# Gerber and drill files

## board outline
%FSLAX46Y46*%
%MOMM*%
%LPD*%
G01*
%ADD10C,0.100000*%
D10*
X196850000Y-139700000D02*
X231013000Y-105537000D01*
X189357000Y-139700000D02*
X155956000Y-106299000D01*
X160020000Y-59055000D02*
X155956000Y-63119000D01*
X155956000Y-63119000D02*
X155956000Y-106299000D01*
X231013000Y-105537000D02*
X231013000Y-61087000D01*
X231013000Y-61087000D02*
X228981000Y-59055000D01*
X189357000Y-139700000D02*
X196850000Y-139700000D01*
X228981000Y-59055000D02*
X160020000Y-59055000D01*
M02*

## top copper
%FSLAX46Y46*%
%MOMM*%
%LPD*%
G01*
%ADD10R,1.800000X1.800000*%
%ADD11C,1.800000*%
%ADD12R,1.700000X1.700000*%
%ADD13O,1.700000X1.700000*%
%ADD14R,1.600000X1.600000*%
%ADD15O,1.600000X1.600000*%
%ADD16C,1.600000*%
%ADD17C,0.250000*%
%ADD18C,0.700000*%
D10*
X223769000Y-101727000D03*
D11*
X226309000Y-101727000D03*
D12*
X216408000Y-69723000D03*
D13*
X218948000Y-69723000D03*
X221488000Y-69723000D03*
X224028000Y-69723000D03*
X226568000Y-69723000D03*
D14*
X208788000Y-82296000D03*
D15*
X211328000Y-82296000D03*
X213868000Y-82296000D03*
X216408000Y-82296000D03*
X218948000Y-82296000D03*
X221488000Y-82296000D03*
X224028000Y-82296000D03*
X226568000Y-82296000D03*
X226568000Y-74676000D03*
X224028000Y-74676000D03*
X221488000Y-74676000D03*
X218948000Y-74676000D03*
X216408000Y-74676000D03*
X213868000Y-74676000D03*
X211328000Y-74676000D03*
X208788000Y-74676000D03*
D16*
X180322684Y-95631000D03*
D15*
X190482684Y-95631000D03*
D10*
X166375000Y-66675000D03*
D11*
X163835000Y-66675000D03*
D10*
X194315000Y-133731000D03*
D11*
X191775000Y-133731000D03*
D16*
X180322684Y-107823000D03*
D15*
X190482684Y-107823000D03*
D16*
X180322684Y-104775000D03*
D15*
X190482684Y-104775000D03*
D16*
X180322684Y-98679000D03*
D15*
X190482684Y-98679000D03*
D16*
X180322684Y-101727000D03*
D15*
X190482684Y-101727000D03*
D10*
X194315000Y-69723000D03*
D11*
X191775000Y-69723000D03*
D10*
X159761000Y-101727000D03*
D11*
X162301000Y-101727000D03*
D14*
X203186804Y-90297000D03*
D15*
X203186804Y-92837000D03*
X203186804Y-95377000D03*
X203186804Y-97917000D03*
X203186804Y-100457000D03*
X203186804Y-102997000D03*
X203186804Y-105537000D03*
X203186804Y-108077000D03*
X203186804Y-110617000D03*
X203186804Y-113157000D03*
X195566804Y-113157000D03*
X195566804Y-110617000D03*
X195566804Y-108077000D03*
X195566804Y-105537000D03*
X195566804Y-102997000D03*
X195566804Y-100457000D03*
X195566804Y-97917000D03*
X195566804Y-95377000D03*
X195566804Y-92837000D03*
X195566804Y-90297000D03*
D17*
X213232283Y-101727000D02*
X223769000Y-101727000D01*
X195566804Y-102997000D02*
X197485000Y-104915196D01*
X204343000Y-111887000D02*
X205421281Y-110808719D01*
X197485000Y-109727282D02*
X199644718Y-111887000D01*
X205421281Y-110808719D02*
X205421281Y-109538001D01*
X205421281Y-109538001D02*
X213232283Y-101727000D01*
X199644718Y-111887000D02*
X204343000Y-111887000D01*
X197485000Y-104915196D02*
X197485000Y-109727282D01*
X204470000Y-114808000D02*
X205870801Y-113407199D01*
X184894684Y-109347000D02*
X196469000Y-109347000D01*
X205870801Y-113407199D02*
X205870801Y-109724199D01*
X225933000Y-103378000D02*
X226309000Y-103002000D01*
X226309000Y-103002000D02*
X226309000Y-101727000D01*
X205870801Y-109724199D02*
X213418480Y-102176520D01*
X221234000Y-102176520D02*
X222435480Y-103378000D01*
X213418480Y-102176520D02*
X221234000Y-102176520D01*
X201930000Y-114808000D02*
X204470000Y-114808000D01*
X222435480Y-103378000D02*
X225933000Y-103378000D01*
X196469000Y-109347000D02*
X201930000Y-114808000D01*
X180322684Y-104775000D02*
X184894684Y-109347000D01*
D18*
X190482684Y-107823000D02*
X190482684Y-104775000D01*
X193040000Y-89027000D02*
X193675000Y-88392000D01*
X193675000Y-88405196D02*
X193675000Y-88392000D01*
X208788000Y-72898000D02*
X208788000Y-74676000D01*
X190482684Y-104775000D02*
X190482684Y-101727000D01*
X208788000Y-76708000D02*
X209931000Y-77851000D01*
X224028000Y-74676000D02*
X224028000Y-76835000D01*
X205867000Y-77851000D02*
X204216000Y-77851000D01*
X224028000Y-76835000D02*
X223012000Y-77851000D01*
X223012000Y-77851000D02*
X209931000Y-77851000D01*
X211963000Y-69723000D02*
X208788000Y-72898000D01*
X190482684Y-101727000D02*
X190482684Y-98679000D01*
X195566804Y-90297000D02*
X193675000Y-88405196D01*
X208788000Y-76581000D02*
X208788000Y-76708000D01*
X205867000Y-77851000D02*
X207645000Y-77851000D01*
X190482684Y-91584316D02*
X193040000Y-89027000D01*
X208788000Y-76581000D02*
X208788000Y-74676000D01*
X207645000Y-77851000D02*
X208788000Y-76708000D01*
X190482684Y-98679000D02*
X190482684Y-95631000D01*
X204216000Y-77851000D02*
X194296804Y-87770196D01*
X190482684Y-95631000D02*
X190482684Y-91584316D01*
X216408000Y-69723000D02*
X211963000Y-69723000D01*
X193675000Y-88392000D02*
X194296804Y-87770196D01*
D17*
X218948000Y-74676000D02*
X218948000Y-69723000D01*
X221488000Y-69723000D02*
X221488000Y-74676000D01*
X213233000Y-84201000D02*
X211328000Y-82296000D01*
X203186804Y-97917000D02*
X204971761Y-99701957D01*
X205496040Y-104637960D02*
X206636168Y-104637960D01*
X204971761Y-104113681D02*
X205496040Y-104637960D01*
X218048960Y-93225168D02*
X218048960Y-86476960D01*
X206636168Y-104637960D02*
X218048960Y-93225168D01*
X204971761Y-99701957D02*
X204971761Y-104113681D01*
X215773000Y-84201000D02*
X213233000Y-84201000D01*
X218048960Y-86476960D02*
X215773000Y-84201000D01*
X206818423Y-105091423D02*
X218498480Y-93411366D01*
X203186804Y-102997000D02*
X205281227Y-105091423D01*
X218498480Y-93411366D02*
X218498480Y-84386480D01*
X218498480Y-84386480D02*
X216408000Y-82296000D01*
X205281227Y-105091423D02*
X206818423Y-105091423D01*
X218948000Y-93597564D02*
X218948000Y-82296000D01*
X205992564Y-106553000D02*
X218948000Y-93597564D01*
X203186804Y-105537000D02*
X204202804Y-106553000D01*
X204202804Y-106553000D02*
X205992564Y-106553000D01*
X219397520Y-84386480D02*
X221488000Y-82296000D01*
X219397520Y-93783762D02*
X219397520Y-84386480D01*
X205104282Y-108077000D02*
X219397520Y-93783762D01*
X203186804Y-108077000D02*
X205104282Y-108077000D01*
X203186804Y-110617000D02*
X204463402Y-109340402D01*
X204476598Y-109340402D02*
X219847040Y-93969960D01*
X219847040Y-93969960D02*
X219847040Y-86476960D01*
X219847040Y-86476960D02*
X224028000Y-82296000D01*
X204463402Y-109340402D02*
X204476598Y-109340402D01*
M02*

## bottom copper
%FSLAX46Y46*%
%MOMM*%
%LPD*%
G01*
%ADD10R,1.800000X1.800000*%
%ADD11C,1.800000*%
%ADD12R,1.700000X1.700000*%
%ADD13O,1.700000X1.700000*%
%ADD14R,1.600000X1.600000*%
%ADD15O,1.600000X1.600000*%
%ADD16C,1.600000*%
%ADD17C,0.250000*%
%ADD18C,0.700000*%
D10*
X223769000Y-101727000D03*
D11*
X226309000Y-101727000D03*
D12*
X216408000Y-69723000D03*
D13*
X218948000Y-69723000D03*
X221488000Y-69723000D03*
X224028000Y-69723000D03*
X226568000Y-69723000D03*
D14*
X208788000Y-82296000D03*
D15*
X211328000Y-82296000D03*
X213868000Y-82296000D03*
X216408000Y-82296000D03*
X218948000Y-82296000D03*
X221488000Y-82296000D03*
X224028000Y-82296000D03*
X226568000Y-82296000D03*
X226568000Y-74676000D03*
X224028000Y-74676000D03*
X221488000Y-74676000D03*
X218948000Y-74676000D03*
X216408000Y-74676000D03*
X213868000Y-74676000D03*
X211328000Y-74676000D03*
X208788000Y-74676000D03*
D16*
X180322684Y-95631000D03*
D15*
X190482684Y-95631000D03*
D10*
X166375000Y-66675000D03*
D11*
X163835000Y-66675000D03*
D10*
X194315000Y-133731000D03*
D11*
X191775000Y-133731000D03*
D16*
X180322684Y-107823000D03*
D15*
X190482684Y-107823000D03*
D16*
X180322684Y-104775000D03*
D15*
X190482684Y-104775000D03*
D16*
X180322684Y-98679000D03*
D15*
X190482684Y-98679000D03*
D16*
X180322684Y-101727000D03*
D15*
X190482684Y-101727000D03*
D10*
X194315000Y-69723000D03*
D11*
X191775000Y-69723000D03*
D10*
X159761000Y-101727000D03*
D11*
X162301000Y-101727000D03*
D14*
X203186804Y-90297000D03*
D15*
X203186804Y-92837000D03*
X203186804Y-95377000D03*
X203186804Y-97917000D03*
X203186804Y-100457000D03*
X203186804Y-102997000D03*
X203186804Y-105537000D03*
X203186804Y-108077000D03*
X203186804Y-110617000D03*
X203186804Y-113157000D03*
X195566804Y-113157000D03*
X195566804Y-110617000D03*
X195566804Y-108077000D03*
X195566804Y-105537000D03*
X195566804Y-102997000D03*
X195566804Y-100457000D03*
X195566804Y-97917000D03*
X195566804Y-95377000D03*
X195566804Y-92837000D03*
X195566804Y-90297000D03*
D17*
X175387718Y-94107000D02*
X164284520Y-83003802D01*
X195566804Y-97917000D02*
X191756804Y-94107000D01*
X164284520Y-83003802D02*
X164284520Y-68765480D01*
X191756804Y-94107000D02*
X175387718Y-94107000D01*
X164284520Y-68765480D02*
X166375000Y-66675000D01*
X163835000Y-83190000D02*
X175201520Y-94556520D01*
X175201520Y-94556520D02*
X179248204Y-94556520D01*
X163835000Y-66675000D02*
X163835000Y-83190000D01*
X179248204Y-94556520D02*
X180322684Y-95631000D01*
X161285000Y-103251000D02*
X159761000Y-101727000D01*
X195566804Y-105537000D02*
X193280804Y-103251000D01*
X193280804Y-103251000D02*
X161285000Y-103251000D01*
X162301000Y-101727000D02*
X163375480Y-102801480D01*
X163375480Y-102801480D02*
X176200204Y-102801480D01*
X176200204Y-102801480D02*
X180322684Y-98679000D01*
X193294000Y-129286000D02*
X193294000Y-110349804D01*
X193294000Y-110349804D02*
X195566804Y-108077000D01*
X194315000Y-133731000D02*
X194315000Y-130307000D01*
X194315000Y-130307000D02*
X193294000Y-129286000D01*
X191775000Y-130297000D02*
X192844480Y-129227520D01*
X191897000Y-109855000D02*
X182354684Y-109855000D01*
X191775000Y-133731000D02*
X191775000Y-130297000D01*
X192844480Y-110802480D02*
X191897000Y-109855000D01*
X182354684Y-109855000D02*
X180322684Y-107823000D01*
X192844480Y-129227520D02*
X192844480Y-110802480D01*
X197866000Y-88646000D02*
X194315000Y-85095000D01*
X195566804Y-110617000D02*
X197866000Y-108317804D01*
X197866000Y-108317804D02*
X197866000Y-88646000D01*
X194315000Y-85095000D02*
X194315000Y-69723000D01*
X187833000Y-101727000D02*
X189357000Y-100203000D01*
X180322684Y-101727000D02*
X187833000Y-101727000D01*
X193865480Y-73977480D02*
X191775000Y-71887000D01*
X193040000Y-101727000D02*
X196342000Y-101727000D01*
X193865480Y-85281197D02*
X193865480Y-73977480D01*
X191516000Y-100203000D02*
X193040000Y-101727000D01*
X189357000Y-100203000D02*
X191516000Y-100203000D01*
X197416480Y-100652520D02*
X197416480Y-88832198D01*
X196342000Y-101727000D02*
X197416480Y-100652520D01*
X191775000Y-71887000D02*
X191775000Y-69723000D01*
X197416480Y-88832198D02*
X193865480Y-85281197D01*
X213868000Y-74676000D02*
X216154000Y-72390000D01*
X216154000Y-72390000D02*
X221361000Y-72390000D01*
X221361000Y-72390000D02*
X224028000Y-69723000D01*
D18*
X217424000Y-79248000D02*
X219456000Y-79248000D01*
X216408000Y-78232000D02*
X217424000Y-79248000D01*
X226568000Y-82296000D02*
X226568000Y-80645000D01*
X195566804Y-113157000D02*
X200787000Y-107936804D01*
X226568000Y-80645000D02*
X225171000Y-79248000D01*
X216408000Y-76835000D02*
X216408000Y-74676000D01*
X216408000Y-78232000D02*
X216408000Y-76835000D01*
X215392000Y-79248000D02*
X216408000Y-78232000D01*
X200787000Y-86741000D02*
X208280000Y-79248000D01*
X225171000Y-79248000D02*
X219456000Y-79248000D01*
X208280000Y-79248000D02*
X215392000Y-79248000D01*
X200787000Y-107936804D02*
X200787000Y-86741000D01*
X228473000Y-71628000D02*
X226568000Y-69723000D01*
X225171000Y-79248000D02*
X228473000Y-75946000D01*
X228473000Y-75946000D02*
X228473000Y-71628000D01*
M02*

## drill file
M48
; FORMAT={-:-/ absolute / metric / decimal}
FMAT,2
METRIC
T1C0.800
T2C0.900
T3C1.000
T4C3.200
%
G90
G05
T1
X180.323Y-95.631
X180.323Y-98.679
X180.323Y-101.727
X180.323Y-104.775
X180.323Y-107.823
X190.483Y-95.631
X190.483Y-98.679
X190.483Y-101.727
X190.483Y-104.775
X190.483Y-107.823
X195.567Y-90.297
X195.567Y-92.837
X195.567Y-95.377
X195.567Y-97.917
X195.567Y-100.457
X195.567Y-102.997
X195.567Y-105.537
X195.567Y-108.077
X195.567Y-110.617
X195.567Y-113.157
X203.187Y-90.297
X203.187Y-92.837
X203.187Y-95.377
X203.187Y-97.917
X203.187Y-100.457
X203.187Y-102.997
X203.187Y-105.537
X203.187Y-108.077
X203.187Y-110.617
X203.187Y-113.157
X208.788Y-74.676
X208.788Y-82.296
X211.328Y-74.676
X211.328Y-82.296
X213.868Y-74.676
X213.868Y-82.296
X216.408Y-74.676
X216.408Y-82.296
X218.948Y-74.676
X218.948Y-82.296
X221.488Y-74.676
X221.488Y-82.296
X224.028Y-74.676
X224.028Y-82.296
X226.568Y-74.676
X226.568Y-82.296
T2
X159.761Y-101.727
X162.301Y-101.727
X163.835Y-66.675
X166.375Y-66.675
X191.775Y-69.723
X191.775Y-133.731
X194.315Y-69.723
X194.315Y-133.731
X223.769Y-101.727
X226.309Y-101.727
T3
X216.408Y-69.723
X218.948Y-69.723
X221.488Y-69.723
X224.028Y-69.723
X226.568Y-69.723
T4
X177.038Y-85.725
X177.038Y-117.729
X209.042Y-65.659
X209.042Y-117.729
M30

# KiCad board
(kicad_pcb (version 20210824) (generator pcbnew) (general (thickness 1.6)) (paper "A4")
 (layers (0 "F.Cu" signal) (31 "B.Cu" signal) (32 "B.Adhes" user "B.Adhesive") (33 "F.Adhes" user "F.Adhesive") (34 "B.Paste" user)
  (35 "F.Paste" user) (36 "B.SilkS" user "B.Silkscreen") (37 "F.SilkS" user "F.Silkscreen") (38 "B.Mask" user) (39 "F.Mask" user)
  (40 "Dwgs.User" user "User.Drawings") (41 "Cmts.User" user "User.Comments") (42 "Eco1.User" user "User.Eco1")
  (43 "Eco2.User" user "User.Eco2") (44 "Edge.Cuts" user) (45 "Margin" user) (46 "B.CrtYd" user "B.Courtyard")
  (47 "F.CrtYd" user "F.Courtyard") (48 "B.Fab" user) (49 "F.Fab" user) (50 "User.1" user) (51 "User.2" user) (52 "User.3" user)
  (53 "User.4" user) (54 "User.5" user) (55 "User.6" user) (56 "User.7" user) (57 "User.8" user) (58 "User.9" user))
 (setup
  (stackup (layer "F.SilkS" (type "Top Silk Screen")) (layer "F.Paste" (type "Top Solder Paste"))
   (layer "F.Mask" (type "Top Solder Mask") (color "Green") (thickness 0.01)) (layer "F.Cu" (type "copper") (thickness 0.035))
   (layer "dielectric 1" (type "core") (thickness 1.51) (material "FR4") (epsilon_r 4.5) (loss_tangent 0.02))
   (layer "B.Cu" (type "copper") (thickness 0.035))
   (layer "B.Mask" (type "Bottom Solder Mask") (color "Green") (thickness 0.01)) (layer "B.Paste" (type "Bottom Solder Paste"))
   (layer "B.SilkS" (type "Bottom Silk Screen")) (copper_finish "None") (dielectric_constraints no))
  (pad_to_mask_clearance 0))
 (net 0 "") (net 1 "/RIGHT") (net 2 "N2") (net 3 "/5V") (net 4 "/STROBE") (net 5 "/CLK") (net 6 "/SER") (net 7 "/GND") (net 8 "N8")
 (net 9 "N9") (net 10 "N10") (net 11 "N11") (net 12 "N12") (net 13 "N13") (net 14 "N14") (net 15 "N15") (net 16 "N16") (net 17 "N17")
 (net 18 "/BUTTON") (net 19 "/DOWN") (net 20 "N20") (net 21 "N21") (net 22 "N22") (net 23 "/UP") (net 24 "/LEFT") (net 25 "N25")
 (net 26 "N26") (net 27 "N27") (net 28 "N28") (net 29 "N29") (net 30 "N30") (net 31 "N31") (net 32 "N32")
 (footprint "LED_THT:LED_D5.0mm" (layer "F.Cu") (at 223.769 101.727)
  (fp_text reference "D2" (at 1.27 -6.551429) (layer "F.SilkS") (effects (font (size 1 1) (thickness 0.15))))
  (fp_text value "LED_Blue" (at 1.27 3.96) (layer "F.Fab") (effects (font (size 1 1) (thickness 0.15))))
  (pad "1" thru_hole rect locked (at 0 0) (size 1.8 1.8) (drill 0.9) (layers *.Cu *.Mask) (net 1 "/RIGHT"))
  (pad "2" thru_hole circle locked (at 2.54 0) (size 1.8 1.8) (drill 0.9) (layers *.Cu *.Mask) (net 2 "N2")))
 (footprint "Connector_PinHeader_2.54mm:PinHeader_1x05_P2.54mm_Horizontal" (layer "F.Cu") (at 216.408 69.723 90)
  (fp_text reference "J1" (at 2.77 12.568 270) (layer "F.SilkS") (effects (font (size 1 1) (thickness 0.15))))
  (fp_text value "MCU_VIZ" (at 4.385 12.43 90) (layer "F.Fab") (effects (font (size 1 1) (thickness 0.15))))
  (pad "1" thru_hole rect locked (at 0 0 90) (size 1.7 1.7) (drill 1) (layers *.Cu *.Mask) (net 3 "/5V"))
  (pad "2" thru_hole oval locked (at 0 2.54 90) (size 1.7 1.7) (drill 1) (layers *.Cu *.Mask) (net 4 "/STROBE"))
  (pad "3" thru_hole oval locked (at 0 5.08 90) (size 1.7 1.7) (drill 1) (layers *.Cu *.Mask) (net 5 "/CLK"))
  (pad "4" thru_hole oval locked (at 0 7.62 90) (size 1.7 1.7) (drill 1) (layers *.Cu *.Mask) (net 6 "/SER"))
  (pad "5" thru_hole oval locked (at 0 10.16 90) (size 1.7 1.7) (drill 1) (layers *.Cu *.Mask) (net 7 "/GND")))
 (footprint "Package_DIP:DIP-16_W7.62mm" (layer "F.Cu") (at 208.788 82.296 90)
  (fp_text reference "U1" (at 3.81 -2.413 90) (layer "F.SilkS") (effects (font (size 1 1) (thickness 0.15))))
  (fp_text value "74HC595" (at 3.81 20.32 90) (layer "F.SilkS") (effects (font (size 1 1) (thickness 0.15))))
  (pad "1" thru_hole rect locked (at 0 0 90) (size 1.6 1.6) (drill 0.8) (layers *.Cu *.Mask) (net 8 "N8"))
  (pad "2" thru_hole oval locked (at 0 2.54 90) (size 1.6 1.6) (drill 0.8) (layers *.Cu *.Mask) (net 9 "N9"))
  (pad "3" thru_hole oval locked (at 0 5.08 90) (size 1.6 1.6) (drill 0.8) (layers *.Cu *.Mask) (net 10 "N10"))
  (pad "4" thru_hole oval locked (at 0 7.62 90) (size 1.6 1.6) (drill 0.8) (layers *.Cu *.Mask) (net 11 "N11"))
  (pad "5" thru_hole oval locked (at 0 10.16 90) (size 1.6 1.6) (drill 0.8) (layers *.Cu *.Mask) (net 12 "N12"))
  (pad "6" thru_hole oval locked (at 0 12.7 90) (size 1.6 1.6) (drill 0.8) (layers *.Cu *.Mask) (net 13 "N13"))
  (pad "7" thru_hole oval locked (at 0 15.24 90) (size 1.6 1.6) (drill 0.8) (layers *.Cu *.Mask) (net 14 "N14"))
  (pad "8" thru_hole oval locked (at 0 17.78 90) (size 1.6 1.6) (drill 0.8) (layers *.Cu *.Mask) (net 7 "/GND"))
  (pad "9" thru_hole oval locked (at 7.62 17.78 90) (size 1.6 1.6) (drill 0.8) (layers *.Cu *.Mask) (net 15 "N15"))
  (pad "10" thru_hole oval locked (at 7.62 15.24 90) (size 1.6 1.6) (drill 0.8) (layers *.Cu *.Mask) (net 3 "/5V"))
  (pad "11" thru_hole oval locked (at 7.62 12.7 90) (size 1.6 1.6) (drill 0.8) (layers *.Cu *.Mask) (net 5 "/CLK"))
  (pad "12" thru_hole oval locked (at 7.62 10.16 90) (size 1.6 1.6) (drill 0.8) (layers *.Cu *.Mask) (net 4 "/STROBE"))
  (pad "13" thru_hole oval locked (at 7.62 7.62 90) (size 1.6 1.6) (drill 0.8) (layers *.Cu *.Mask) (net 7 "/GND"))
  (pad "14" thru_hole oval locked (at 7.62 5.08 90) (size 1.6 1.6) (drill 0.8) (layers *.Cu *.Mask) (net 6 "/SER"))
  (pad "15" thru_hole oval locked (at 7.62 2.54 90) (size 1.6 1.6) (drill 0.8) (layers *.Cu *.Mask) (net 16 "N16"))
  (pad "16" thru_hole oval locked (at 7.62 0 90) (size 1.6 1.6) (drill 0.8) (layers *.Cu *.Mask) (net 3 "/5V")))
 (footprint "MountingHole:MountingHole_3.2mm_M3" (layer "F.Cu") (at 177.038 117.729)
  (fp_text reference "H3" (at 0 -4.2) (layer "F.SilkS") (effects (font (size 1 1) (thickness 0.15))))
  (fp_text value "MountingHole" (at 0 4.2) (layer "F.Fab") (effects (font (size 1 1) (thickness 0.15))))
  (pad "" np_thru_hole circle locked (at 0 0) (size 3.2 3.2) (drill 3.2) (layers *.Cu *.Mask)))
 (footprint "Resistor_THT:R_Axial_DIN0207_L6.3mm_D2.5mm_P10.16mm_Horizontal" (layer "F.Cu") (at 180.322684 95.631)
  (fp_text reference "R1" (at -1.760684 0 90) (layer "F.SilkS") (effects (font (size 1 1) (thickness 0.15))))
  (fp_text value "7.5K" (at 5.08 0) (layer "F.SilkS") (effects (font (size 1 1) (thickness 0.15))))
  (pad "1" thru_hole circle locked (at 0 0) (size 1.6 1.6) (drill 0.8) (layers *.Cu *.Mask) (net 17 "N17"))
  (pad "2" thru_hole oval locked (at 10.16 0) (size 1.6 1.6) (drill 0.8) (layers *.Cu *.Mask) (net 3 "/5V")))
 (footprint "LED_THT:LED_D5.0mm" (layer "F.Cu") (at 166.375 66.675 180)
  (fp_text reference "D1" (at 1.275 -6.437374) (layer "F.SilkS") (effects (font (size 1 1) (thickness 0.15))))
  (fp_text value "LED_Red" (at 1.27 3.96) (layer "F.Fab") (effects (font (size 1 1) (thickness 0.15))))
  (pad "1" thru_hole rect locked (at 0 0 180) (size 1.8 1.8) (drill 0.9) (layers *.Cu *.Mask) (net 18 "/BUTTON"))
  (pad "2" thru_hole circle locked (at 2.54 0 180) (size 1.8 1.8) (drill 0.9) (layers *.Cu *.Mask) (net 17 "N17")))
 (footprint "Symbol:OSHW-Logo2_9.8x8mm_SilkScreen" (layer "F.Cu") (at 187.325 85.725)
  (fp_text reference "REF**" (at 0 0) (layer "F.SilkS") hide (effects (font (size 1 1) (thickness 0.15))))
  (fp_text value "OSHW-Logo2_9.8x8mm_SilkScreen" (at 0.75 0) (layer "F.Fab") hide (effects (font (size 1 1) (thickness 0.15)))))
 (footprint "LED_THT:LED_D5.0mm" (layer "F.Cu") (at 194.315 133.731 180)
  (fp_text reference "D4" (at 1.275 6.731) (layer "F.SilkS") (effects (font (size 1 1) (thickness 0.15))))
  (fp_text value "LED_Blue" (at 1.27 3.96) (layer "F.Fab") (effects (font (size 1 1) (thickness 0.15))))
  (pad "1" thru_hole rect locked (at 0 0 180) (size 1.8 1.8) (drill 0.9) (layers *.Cu *.Mask) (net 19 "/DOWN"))
  (pad "2" thru_hole circle locked (at 2.54 0 180) (size 1.8 1.8) (drill 0.9) (layers *.Cu *.Mask) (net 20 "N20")))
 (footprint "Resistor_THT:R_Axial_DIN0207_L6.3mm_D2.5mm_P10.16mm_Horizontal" (layer "F.Cu") (at 180.322684 107.823)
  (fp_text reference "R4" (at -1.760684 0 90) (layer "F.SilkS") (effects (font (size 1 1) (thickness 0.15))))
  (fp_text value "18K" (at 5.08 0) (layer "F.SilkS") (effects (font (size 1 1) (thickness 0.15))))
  (pad "1" thru_hole circle locked (at 0 0) (size 1.6 1.6) (drill 0.8) (layers *.Cu *.Mask) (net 20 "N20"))
  (pad "2" thru_hole oval locked (at 10.16 0) (size 1.6 1.6) (drill 0.8) (layers *.Cu *.Mask) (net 3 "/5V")))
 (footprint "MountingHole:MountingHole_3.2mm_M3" (layer "F.Cu") (at 209.042 117.729)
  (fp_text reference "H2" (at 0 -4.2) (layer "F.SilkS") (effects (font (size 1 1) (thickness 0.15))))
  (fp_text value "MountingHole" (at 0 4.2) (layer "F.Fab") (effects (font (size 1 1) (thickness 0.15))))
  (pad "" np_thru_hole circle locked (at 0 0) (size 3.2 3.2) (drill 3.2) (layers *.Cu *.Mask)))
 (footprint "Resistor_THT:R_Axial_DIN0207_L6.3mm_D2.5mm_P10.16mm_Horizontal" (layer "F.Cu") (at 180.322684 104.775)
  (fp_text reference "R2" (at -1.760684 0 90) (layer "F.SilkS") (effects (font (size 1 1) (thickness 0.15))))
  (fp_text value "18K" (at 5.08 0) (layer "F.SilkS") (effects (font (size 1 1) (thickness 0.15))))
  (pad "1" thru_hole circle locked (at 0 0) (size 1.6 1.6) (drill 0.8) (layers *.Cu *.Mask) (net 2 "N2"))
  (pad "2" thru_hole oval locked (at 10.16 0) (size 1.6 1.6) (drill 0.8) (layers *.Cu *.Mask) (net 3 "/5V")))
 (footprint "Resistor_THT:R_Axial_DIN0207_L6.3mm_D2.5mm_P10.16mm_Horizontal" (layer "F.Cu") (at 180.322684 98.679)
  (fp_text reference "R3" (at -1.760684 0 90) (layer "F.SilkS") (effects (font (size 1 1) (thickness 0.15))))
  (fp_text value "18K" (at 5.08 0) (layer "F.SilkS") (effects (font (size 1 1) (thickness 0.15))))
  (pad "1" thru_hole circle locked (at 0 0) (size 1.6 1.6) (drill 0.8) (layers *.Cu *.Mask) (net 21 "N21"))
  (pad "2" thru_hole oval locked (at 10.16 0) (size 1.6 1.6) (drill 0.8) (layers *.Cu *.Mask) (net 3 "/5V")))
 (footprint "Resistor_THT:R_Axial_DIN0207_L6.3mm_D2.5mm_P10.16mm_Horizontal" (layer "F.Cu") (at 180.322684 101.727)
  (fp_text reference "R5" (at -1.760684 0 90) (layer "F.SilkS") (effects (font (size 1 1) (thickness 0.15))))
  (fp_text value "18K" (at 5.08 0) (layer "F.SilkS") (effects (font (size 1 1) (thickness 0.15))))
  (pad "1" thru_hole circle locked (at 0 0) (size 1.6 1.6) (drill 0.8) (layers *.Cu *.Mask) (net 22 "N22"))
  (pad "2" thru_hole oval locked (at 10.16 0) (size 1.6 1.6) (drill 0.8) (layers *.Cu *.Mask) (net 3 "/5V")))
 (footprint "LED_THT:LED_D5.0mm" (layer "F.Cu") (at 194.315 69.723 180)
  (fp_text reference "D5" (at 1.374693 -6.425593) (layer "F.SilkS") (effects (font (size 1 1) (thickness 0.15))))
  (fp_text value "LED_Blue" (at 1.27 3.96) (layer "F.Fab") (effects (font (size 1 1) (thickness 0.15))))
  (pad "1" thru_hole rect locked (at 0 0 180) (size 1.8 1.8) (drill 0.9) (layers *.Cu *.Mask) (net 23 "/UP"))
  (pad "2" thru_hole circle locked (at 2.54 0 180) (size 1.8 1.8) (drill 0.9) (layers *.Cu *.Mask) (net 22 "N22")))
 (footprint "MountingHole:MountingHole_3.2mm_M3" (layer "F.Cu") (at 209.042 65.659)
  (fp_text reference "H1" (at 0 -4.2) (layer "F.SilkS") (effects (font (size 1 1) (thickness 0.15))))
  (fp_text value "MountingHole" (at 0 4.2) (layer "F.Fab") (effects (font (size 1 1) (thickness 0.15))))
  (pad "" np_thru_hole circle locked (at 0 0) (size 3.2 3.2) (drill 3.2) (layers *.Cu *.Mask)))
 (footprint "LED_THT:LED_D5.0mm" (layer "F.Cu") (at 159.761 101.727)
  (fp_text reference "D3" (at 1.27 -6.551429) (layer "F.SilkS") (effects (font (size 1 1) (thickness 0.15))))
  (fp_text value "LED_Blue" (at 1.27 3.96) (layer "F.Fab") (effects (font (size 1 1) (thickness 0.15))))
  (pad "1" thru_hole rect locked (at 0 0) (size 1.8 1.8) (drill 0.9) (layers *.Cu *.Mask) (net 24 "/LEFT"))
  (pad "2" thru_hole circle locked (at 2.54 0) (size 1.8 1.8) (drill 0.9) (layers *.Cu *.Mask) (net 21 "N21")))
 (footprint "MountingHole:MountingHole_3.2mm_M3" (layer "F.Cu") (at 177.038 85.725)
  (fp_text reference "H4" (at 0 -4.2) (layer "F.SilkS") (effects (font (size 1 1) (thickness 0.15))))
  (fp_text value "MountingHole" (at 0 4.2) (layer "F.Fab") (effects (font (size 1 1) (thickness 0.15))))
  (pad "" np_thru_hole circle locked (at 0 0) (size 3.2 3.2) (drill 3.2) (layers *.Cu *.Mask)))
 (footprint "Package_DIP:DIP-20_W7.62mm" (layer "B.Cu") (at 203.186804 90.297 180)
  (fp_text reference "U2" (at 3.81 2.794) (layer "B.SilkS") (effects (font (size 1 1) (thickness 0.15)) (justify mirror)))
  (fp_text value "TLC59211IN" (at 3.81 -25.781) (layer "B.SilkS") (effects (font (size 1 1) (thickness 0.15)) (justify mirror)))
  (pad "1" thru_hole rect locked (at 0 0 180) (size 1.6 1.6) (drill 0.8) (layers *.Cu *.Mask) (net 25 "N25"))
  (pad "2" thru_hole oval locked (at 0 -2.54 180) (size 1.6 1.6) (drill 0.8) (layers *.Cu *.Mask) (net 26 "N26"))
  (pad "3" thru_hole oval locked (at 0 -5.08 180) (size 1.6 1.6) (drill 0.8) (layers *.Cu *.Mask) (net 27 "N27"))
  (pad "4" thru_hole oval locked (at 0 -7.62 180) (size 1.6 1.6) (drill 0.8) (layers *.Cu *.Mask) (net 9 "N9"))
  (pad "5" thru_hole oval locked (at 0 -10.16 180) (size 1.6 1.6) (drill 0.8) (layers *.Cu *.Mask) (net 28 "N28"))
  (pad "6" thru_hole oval locked (at 0 -12.7 180) (size 1.6 1.6) (drill 0.8) (layers *.Cu *.Mask) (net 11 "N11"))
  (pad "7" thru_hole oval locked (at 0 -15.24 180) (size 1.6 1.6) (drill 0.8) (layers *.Cu *.Mask) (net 12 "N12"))
  (pad "8" thru_hole oval locked (at 0 -17.78 180) (size 1.6 1.6) (drill 0.8) (layers *.Cu *.Mask) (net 13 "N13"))
  (pad "9" thru_hole oval locked (at 0 -20.32 180) (size 1.6 1.6) (drill 0.8) (layers *.Cu *.Mask) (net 14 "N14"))
  (pad "10" thru_hole oval locked (at 0 -22.86 180) (size 1.6 1.6) (drill 0.8) (layers *.Cu *.Mask) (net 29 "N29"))
  (pad "11" thru_hole oval locked (at 7.62 -22.86 180) (size 1.6 1.6) (drill 0.8) (layers *.Cu *.Mask) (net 7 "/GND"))
  (pad "12" thru_hole oval locked (at 7.62 -20.32 180) (size 1.6 1.6) (drill 0.8) (layers *.Cu *.Mask) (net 23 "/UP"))
  (pad "13" thru_hole oval locked (at 7.62 -17.78 180) (size 1.6 1.6) (drill 0.8) (layers *.Cu *.Mask) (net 19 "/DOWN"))
  (pad "14" thru_hole oval locked (at 7.62 -15.24 180) (size 1.6 1.6) (drill 0.8) (layers *.Cu *.Mask) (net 24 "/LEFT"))
  (pad "15" thru_hole oval locked (at 7.62 -12.7 180) (size 1.6 1.6) (drill 0.8) (layers *.Cu *.Mask) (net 1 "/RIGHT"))
  (pad "16" thru_hole oval locked (at 7.62 -10.16 180) (size 1.6 1.6) (drill 0.8) (layers *.Cu *.Mask) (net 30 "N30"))
  (pad "17" thru_hole oval locked (at 7.62 -7.62 180) (size 1.6 1.6) (drill 0.8) (layers *.Cu *.Mask) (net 18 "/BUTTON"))
  (pad "18" thru_hole oval locked (at 7.62 -5.08 180) (size 1.6 1.6) (drill 0.8) (layers *.Cu *.Mask) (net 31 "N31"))
  (pad "19" thru_hole oval locked (at 7.62 -2.54 180) (size 1.6 1.6) (drill 0.8) (layers *.Cu *.Mask) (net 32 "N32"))
  (pad "20" thru_hole oval locked (at 7.62 0 180) (size 1.6 1.6) (drill 0.8) (layers *.Cu *.Mask) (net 3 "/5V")))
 (gr_line (start 196.85 139.7) (end 231.013 105.537) (layer "Edge.Cuts") (width 0.1))
 (gr_line (start 189.357 139.7) (end 155.956 106.299) (layer "Edge.Cuts") (width 0.1))
 (gr_line (start 160.02 59.055) (end 155.956 63.119) (layer "Edge.Cuts") (width 0.1))
 (gr_line (start 155.956 63.119) (end 155.956 106.299) (layer "Edge.Cuts") (width 0.1))
 (gr_line (start 231.013 105.537) (end 231.013 61.087) (layer "Edge.Cuts") (width 0.1))
 (gr_line (start 231.013 61.087) (end 228.981 59.055) (layer "Edge.Cuts") (width 0.1))
 (gr_line (start 189.357 139.7) (end 196.85 139.7) (layer "Edge.Cuts") (width 0.1))
 (gr_line (start 228.981 59.055) (end 160.02 59.055) (layer "Edge.Cuts") (width 0.1))
 (segment (start 175.387718 94.107) (end 164.28452 83.003802) (width 0.25) (layer "B.Cu") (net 18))
 (segment (start 195.566804 97.917) (end 191.756804 94.107) (width 0.25) (layer "B.Cu") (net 18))
 (segment (start 164.28452 83.003802) (end 164.28452 68.76548) (width 0.25) (layer "B.Cu") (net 18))
 (segment (start 191.756804 94.107) (end 175.387718 94.107) (width 0.25) (layer "B.Cu") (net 18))
 (segment (start 164.28452 68.76548) (end 166.375 66.675) (width 0.25) (layer "B.Cu") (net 18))
 (segment (start 163.835 83.19) (end 175.20152 94.55652) (width 0.25) (layer "B.Cu") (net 17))
 (segment (start 175.20152 94.55652) (end 179.248204 94.55652) (width 0.25) (layer "B.Cu") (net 17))
 (segment (start 163.835 66.675) (end 163.835 83.19) (width 0.25) (layer "B.Cu") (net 17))
 (segment (start 179.248204 94.55652) (end 180.322684 95.631) (width 0.25) (layer "B.Cu") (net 17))
 (segment (start 213.232283 101.727) (end 223.769 101.727) (width 0.25) (layer "F.Cu") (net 1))
 (segment (start 195.566804 102.997) (end 197.485 104.915196) (width 0.25) (layer "F.Cu") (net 1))
 (segment (start 204.343 111.887) (end 205.421281 110.808719) (width 0.25) (layer "F.Cu") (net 1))
 (segment (start 197.485 109.727282) (end 199.644718 111.887) (width 0.25) (layer "F.Cu") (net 1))
 (segment (start 205.421281 110.808719) (end 205.421281 109.538001) (width 0.25) (layer "F.Cu") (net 1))
 (segment (start 205.421281 109.538001) (end 213.232283 101.727) (width 0.25) (layer "F.Cu") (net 1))
 (segment (start 199.644718 111.887) (end 204.343 111.887) (width 0.25) (layer "F.Cu") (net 1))
 (segment (start 197.485 104.915196) (end 197.485 109.727282) (width 0.25) (layer "F.Cu") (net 1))
 (segment (start 204.47 114.808) (end 205.870801 113.407199) (width 0.25) (layer "F.Cu") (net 2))
 (segment (start 184.894684 109.347) (end 196.469 109.347) (width 0.25) (layer "F.Cu") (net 2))
 (segment (start 205.870801 113.407199) (end 205.870801 109.724199) (width 0.25) (layer "F.Cu") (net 2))
 (segment (start 225.933 103.378) (end 226.309 103.002) (width 0.25) (layer "F.Cu") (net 2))
 (segment (start 226.309 103.002) (end 226.309 101.727) (width 0.25) (layer "F.Cu") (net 2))
 (segment (start 205.870801 109.724199) (end 213.41848 102.17652) (width 0.25) (layer "F.Cu") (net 2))
 (segment (start 221.234 102.17652) (end 222.43548 103.378) (width 0.25) (layer "F.Cu") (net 2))
 (segment (start 213.41848 102.17652) (end 221.234 102.17652) (width 0.25) (layer "F.Cu") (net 2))
 (segment (start 201.93 114.808) (end 204.47 114.808) (width 0.25) (layer "F.Cu") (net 2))
 (segment (start 222.43548 103.378) (end 225.933 103.378) (width 0.25) (layer "F.Cu") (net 2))
 (segment (start 196.469 109.347) (end 201.93 114.808) (width 0.25) (layer "F.Cu") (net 2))
 (segment (start 180.322684 104.775) (end 184.894684 109.347) (width 0.25) (layer "F.Cu") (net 2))
 (segment (start 161.285 103.251) (end 159.761 101.727) (width 0.25) (layer "B.Cu") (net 24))
 (segment (start 195.566804 105.537) (end 193.280804 103.251) (width 0.25) (layer "B.Cu") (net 24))
 (segment (start 193.280804 103.251) (end 161.285 103.251) (width 0.25) (layer "B.Cu") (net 24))
 (segment (start 162.301 101.727) (end 163.37548 102.80148) (width 0.25) (layer "B.Cu") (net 21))
 (segment (start 163.37548 102.80148) (end 176.200204 102.80148) (width 0.25) (layer "B.Cu") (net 21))
 (segment (start 176.200204 102.80148) (end 180.322684 98.679) (width 0.25) (layer "B.Cu") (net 21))
 (segment (start 193.294 129.286) (end 193.294 110.349804) (width 0.25) (layer "B.Cu") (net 19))
 (segment (start 193.294 110.349804) (end 195.566804 108.077) (width 0.25) (layer "B.Cu") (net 19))
 (segment (start 194.315 133.731) (end 194.315 130.307) (width 0.25) (layer "B.Cu") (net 19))
 (segment (start 194.315 130.307) (end 193.294 129.286) (width 0.25) (layer "B.Cu") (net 19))
 (segment (start 191.775 130.297) (end 192.84448 129.22752) (width 0.25) (layer "B.Cu") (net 20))
 (segment (start 191.897 109.855) (end 182.354684 109.855) (width 0.25) (layer "B.Cu") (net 20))
 (segment (start 191.775 133.731) (end 191.775 130.297) (width 0.25) (layer "B.Cu") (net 20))
 (segment (start 192.84448 110.80248) (end 191.897 109.855) (width 0.25) (layer "B.Cu") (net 20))
 (segment (start 182.354684 109.855) (end 180.322684 107.823) (width 0.25) (layer "B.Cu") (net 20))
 (segment (start 192.84448 129.22752) (end 192.84448 110.80248) (width 0.25) (layer "B.Cu") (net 20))
 (segment (start 197.866 88.646) (end 194.315 85.095) (width 0.25) (layer "B.Cu") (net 23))
 (segment (start 195.566804 110.617) (end 197.866 108.317804) (width 0.25) (layer "B.Cu") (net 23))
 (segment (start 197.866 108.317804) (end 197.866 88.646) (width 0.25) (layer "B.Cu") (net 23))
 (segment (start 194.315 85.095) (end 194.315 69.723) (width 0.25) (layer "B.Cu") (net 23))
 (segment (start 187.833 101.727) (end 189.357 100.203) (width 0.25) (layer "B.Cu") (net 22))
 (segment (start 180.322684 101.727) (end 187.833 101.727) (width 0.25) (layer "B.Cu") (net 22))
 (segment (start 193.86548 73.97748) (end 191.775 71.887) (width 0.25) (layer "B.Cu") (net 22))
 (segment (start 193.04 101.727) (end 196.342 101.727) (width 0.25) (layer "B.Cu") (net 22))
 (segment (start 193.86548 85.281197) (end 193.86548 73.97748) (width 0.25) (layer "B.Cu") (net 22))
 (segment (start 191.516 100.203) (end 193.04 101.727) (width 0.25) (layer "B.Cu") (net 22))
 (segment (start 189.357 100.203) (end 191.516 100.203) (width 0.25) (layer "B.Cu") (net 22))
 (segment (start 197.41648 100.65252) (end 197.41648 88.832198) (width 0.25) (layer "B.Cu") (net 22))
 (segment (start 196.342 101.727) (end 197.41648 100.65252) (width 0.25) (layer "B.Cu") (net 22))
 (segment (start 191.775 71.887) (end 191.775 69.723) (width 0.25) (layer "B.Cu") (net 22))
 (segment (start 197.41648 88.832198) (end 193.86548 85.281197) (width 0.25) (layer "B.Cu") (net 22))
 (segment (start 190.482684 107.823) (end 190.482684 104.775) (width 0.7) (layer "F.Cu") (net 3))
 (segment (start 193.04 89.027) (end 193.675 88.392) (width 0.7) (layer "F.Cu") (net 3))
 (segment (start 193.675 88.405196) (end 193.675 88.392) (width 0.7) (layer "F.Cu") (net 3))
 (segment (start 208.788 72.898) (end 208.788 74.676) (width 0.7) (layer "F.Cu") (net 3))
 (segment (start 190.482684 104.775) (end 190.482684 101.727) (width 0.7) (layer "F.Cu") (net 3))
 (segment (start 208.788 76.708) (end 209.931 77.851) (width 0.7) (layer "F.Cu") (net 3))
 (segment (start 224.028 74.676) (end 224.028 76.835) (width 0.7) (layer "F.Cu") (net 3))
 (segment (start 205.867 77.851) (end 204.216 77.851) (width 0.7) (layer "F.Cu") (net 3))
 (segment (start 224.028 76.835) (end 223.012 77.851) (width 0.7) (layer "F.Cu") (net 3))
 (segment (start 223.012 77.851) (end 209.931 77.851) (width 0.7) (layer "F.Cu") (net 3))
 (segment (start 211.963 69.723) (end 208.788 72.898) (width 0.7) (layer "F.Cu") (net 3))
 (segment (start 190.482684 101.727) (end 190.482684 98.679) (width 0.7) (layer "F.Cu") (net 3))
 (segment (start 195.566804 90.297) (end 193.675 88.405196) (width 0.7) (layer "F.Cu") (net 3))
 (segment (start 208.788 76.581) (end 208.788 76.708) (width 0.7) (layer "F.Cu") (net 3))
 (segment (start 205.867 77.851) (end 207.645 77.851) (width 0.7) (layer "F.Cu") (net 3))
 (segment (start 190.482684 91.584316) (end 193.04 89.027) (width 0.7) (layer "F.Cu") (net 3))
 (segment (start 208.788 76.581) (end 208.788 74.676) (width 0.7) (layer "F.Cu") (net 3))
 (segment (start 207.645 77.851) (end 208.788 76.708) (width 0.7) (layer "F.Cu") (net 3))
 (segment (start 190.482684 98.679) (end 190.482684 95.631) (width 0.7) (layer "F.Cu") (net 3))
 (segment (start 204.216 77.851) (end 194.296804 87.770196) (width 0.7) (layer "F.Cu") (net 3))
 (segment (start 190.482684 95.631) (end 190.482684 91.584316) (width 0.7) (layer "F.Cu") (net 3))
 (segment (start 216.408 69.723) (end 211.963 69.723) (width 0.7) (layer "F.Cu") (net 3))
 (segment (start 193.675 88.392) (end 194.296804 87.770196) (width 0.7) (layer "F.Cu") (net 3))
 (segment (start 218.948 74.676) (end 218.948 69.723) (width 0.25) (layer "F.Cu") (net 4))
 (segment (start 221.488 69.723) (end 221.488 74.676) (width 0.25) (layer "F.Cu") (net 5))
 (segment (start 213.868 74.676) (end 216.154 72.39) (width 0.25) (layer "B.Cu") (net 6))
 (segment (start 216.154 72.39) (end 221.361 72.39) (width 0.25) (layer "B.Cu") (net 6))
 (segment (start 221.361 72.39) (end 224.028 69.723) (width 0.25) (layer "B.Cu") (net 6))
 (segment (start 217.424 79.248) (end 219.456 79.248) (width 0.7) (layer "B.Cu") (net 7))
 (segment (start 216.408 78.232) (end 217.424 79.248) (width 0.7) (layer "B.Cu") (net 7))
 (segment (start 226.568 82.296) (end 226.568 80.645) (width 0.7) (layer "B.Cu") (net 7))
 (segment (start 195.566804 113.157) (end 200.787 107.936804) (width 0.7) (layer "B.Cu") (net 7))
 (segment (start 226.568 80.645) (end 225.171 79.248) (width 0.7) (layer "B.Cu") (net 7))
 (segment (start 216.408 76.835) (end 216.408 74.676) (width 0.7) (layer "B.Cu") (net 7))
 (segment (start 216.408 78.232) (end 216.408 76.835) (width 0.7) (layer "B.Cu") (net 7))
 (segment (start 215.392 79.248) (end 216.408 78.232) (width 0.7) (layer "B.Cu") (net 7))
 (segment (start 200.787 86.741) (end 208.28 79.248) (width 0.7) (layer "B.Cu") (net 7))
 (segment (start 225.171 79.248) (end 219.456 79.248) (width 0.7) (layer "B.Cu") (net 7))
 (segment (start 208.28 79.248) (end 215.392 79.248) (width 0.7) (layer "B.Cu") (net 7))
 (segment (start 200.787 107.936804) (end 200.787 86.741) (width 0.7) (layer "B.Cu") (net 7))
 (segment (start 228.473 71.628) (end 226.568 69.723) (width 0.7) (layer "B.Cu") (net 7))
 (segment (start 225.171 79.248) (end 228.473 75.946) (width 0.7) (layer "B.Cu") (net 7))
 (segment (start 228.473 75.946) (end 228.473 71.628) (width 0.7) (layer "B.Cu") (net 7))
 (segment (start 213.233 84.201) (end 211.328 82.296) (width 0.25) (layer "F.Cu") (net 9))
 (segment (start 203.186804 97.917) (end 204.971761 99.701957) (width 0.25) (layer "F.Cu") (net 9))
 (segment (start 205.49604 104.63796) (end 206.636168 104.63796) (width 0.25) (layer "F.Cu") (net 9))
 (segment (start 204.971761 104.113681) (end 205.49604 104.63796) (width 0.25) (layer "F.Cu") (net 9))
 (segment (start 218.04896 93.225168) (end 218.04896 86.47696) (width 0.25) (layer "F.Cu") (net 9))
 (segment (start 206.636168 104.63796) (end 218.04896 93.225168) (width 0.25) (layer "F.Cu") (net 9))
 (segment (start 204.971761 99.701957) (end 204.971761 104.113681) (width 0.25) (layer "F.Cu") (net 9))
 (segment (start 215.773 84.201) (end 213.233 84.201) (width 0.25) (layer "F.Cu") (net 9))
 (segment (start 218.04896 86.47696) (end 215.773 84.201) (width 0.25) (layer "F.Cu") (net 9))
 (segment (start 206.818423 105.091423) (end 218.49848 93.411366) (width 0.25) (layer "F.Cu") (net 11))
 (segment (start 203.186804 102.997) (end 205.281227 105.091423) (width 0.25) (layer "F.Cu") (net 11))
 (segment (start 218.49848 93.411366) (end 218.49848 84.38648) (width 0.25) (layer "F.Cu") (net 11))
 (segment (start 218.49848 84.38648) (end 216.408 82.296) (width 0.25) (layer "F.Cu") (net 11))
 (segment (start 205.281227 105.091423) (end 206.818423 105.091423) (width 0.25) (layer "F.Cu") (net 11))
 (segment (start 218.948 93.597564) (end 218.948 82.296) (width 0.25) (layer "F.Cu") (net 12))
 (segment (start 205.992564 106.553) (end 218.948 93.597564) (width 0.25) (layer "F.Cu") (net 12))
 (segment (start 203.186804 105.537) (end 204.202804 106.553) (width 0.25) (layer "F.Cu") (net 12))
 (segment (start 204.202804 106.553) (end 205.992564 106.553) (width 0.25) (layer "F.Cu") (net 12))
 (segment (start 219.39752 84.38648) (end 221.488 82.296) (width 0.25) (layer "F.Cu") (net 13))
 (segment (start 219.39752 93.783762) (end 219.39752 84.38648) (width 0.25) (layer "F.Cu") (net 13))
 (segment (start 205.104282 108.077) (end 219.39752 93.783762) (width 0.25) (layer "F.Cu") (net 13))
 (segment (start 203.186804 108.077) (end 205.104282 108.077) (width 0.25) (layer "F.Cu") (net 13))
 (segment (start 203.186804 110.617) (end 204.463402 109.340402) (width 0.25) (layer "F.Cu") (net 14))
 (segment (start 204.476598 109.340402) (end 219.84704 93.96996) (width 0.25) (layer "F.Cu") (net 14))
 (segment (start 219.84704 93.96996) (end 219.84704 86.47696) (width 0.25) (layer "F.Cu") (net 14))
 (segment (start 219.84704 86.47696) (end 224.028 82.296) (width 0.25) (layer "F.Cu") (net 14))
 (segment (start 204.463402 109.340402) (end 204.476598 109.340402) (width 0.25) (layer "F.Cu") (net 14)))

